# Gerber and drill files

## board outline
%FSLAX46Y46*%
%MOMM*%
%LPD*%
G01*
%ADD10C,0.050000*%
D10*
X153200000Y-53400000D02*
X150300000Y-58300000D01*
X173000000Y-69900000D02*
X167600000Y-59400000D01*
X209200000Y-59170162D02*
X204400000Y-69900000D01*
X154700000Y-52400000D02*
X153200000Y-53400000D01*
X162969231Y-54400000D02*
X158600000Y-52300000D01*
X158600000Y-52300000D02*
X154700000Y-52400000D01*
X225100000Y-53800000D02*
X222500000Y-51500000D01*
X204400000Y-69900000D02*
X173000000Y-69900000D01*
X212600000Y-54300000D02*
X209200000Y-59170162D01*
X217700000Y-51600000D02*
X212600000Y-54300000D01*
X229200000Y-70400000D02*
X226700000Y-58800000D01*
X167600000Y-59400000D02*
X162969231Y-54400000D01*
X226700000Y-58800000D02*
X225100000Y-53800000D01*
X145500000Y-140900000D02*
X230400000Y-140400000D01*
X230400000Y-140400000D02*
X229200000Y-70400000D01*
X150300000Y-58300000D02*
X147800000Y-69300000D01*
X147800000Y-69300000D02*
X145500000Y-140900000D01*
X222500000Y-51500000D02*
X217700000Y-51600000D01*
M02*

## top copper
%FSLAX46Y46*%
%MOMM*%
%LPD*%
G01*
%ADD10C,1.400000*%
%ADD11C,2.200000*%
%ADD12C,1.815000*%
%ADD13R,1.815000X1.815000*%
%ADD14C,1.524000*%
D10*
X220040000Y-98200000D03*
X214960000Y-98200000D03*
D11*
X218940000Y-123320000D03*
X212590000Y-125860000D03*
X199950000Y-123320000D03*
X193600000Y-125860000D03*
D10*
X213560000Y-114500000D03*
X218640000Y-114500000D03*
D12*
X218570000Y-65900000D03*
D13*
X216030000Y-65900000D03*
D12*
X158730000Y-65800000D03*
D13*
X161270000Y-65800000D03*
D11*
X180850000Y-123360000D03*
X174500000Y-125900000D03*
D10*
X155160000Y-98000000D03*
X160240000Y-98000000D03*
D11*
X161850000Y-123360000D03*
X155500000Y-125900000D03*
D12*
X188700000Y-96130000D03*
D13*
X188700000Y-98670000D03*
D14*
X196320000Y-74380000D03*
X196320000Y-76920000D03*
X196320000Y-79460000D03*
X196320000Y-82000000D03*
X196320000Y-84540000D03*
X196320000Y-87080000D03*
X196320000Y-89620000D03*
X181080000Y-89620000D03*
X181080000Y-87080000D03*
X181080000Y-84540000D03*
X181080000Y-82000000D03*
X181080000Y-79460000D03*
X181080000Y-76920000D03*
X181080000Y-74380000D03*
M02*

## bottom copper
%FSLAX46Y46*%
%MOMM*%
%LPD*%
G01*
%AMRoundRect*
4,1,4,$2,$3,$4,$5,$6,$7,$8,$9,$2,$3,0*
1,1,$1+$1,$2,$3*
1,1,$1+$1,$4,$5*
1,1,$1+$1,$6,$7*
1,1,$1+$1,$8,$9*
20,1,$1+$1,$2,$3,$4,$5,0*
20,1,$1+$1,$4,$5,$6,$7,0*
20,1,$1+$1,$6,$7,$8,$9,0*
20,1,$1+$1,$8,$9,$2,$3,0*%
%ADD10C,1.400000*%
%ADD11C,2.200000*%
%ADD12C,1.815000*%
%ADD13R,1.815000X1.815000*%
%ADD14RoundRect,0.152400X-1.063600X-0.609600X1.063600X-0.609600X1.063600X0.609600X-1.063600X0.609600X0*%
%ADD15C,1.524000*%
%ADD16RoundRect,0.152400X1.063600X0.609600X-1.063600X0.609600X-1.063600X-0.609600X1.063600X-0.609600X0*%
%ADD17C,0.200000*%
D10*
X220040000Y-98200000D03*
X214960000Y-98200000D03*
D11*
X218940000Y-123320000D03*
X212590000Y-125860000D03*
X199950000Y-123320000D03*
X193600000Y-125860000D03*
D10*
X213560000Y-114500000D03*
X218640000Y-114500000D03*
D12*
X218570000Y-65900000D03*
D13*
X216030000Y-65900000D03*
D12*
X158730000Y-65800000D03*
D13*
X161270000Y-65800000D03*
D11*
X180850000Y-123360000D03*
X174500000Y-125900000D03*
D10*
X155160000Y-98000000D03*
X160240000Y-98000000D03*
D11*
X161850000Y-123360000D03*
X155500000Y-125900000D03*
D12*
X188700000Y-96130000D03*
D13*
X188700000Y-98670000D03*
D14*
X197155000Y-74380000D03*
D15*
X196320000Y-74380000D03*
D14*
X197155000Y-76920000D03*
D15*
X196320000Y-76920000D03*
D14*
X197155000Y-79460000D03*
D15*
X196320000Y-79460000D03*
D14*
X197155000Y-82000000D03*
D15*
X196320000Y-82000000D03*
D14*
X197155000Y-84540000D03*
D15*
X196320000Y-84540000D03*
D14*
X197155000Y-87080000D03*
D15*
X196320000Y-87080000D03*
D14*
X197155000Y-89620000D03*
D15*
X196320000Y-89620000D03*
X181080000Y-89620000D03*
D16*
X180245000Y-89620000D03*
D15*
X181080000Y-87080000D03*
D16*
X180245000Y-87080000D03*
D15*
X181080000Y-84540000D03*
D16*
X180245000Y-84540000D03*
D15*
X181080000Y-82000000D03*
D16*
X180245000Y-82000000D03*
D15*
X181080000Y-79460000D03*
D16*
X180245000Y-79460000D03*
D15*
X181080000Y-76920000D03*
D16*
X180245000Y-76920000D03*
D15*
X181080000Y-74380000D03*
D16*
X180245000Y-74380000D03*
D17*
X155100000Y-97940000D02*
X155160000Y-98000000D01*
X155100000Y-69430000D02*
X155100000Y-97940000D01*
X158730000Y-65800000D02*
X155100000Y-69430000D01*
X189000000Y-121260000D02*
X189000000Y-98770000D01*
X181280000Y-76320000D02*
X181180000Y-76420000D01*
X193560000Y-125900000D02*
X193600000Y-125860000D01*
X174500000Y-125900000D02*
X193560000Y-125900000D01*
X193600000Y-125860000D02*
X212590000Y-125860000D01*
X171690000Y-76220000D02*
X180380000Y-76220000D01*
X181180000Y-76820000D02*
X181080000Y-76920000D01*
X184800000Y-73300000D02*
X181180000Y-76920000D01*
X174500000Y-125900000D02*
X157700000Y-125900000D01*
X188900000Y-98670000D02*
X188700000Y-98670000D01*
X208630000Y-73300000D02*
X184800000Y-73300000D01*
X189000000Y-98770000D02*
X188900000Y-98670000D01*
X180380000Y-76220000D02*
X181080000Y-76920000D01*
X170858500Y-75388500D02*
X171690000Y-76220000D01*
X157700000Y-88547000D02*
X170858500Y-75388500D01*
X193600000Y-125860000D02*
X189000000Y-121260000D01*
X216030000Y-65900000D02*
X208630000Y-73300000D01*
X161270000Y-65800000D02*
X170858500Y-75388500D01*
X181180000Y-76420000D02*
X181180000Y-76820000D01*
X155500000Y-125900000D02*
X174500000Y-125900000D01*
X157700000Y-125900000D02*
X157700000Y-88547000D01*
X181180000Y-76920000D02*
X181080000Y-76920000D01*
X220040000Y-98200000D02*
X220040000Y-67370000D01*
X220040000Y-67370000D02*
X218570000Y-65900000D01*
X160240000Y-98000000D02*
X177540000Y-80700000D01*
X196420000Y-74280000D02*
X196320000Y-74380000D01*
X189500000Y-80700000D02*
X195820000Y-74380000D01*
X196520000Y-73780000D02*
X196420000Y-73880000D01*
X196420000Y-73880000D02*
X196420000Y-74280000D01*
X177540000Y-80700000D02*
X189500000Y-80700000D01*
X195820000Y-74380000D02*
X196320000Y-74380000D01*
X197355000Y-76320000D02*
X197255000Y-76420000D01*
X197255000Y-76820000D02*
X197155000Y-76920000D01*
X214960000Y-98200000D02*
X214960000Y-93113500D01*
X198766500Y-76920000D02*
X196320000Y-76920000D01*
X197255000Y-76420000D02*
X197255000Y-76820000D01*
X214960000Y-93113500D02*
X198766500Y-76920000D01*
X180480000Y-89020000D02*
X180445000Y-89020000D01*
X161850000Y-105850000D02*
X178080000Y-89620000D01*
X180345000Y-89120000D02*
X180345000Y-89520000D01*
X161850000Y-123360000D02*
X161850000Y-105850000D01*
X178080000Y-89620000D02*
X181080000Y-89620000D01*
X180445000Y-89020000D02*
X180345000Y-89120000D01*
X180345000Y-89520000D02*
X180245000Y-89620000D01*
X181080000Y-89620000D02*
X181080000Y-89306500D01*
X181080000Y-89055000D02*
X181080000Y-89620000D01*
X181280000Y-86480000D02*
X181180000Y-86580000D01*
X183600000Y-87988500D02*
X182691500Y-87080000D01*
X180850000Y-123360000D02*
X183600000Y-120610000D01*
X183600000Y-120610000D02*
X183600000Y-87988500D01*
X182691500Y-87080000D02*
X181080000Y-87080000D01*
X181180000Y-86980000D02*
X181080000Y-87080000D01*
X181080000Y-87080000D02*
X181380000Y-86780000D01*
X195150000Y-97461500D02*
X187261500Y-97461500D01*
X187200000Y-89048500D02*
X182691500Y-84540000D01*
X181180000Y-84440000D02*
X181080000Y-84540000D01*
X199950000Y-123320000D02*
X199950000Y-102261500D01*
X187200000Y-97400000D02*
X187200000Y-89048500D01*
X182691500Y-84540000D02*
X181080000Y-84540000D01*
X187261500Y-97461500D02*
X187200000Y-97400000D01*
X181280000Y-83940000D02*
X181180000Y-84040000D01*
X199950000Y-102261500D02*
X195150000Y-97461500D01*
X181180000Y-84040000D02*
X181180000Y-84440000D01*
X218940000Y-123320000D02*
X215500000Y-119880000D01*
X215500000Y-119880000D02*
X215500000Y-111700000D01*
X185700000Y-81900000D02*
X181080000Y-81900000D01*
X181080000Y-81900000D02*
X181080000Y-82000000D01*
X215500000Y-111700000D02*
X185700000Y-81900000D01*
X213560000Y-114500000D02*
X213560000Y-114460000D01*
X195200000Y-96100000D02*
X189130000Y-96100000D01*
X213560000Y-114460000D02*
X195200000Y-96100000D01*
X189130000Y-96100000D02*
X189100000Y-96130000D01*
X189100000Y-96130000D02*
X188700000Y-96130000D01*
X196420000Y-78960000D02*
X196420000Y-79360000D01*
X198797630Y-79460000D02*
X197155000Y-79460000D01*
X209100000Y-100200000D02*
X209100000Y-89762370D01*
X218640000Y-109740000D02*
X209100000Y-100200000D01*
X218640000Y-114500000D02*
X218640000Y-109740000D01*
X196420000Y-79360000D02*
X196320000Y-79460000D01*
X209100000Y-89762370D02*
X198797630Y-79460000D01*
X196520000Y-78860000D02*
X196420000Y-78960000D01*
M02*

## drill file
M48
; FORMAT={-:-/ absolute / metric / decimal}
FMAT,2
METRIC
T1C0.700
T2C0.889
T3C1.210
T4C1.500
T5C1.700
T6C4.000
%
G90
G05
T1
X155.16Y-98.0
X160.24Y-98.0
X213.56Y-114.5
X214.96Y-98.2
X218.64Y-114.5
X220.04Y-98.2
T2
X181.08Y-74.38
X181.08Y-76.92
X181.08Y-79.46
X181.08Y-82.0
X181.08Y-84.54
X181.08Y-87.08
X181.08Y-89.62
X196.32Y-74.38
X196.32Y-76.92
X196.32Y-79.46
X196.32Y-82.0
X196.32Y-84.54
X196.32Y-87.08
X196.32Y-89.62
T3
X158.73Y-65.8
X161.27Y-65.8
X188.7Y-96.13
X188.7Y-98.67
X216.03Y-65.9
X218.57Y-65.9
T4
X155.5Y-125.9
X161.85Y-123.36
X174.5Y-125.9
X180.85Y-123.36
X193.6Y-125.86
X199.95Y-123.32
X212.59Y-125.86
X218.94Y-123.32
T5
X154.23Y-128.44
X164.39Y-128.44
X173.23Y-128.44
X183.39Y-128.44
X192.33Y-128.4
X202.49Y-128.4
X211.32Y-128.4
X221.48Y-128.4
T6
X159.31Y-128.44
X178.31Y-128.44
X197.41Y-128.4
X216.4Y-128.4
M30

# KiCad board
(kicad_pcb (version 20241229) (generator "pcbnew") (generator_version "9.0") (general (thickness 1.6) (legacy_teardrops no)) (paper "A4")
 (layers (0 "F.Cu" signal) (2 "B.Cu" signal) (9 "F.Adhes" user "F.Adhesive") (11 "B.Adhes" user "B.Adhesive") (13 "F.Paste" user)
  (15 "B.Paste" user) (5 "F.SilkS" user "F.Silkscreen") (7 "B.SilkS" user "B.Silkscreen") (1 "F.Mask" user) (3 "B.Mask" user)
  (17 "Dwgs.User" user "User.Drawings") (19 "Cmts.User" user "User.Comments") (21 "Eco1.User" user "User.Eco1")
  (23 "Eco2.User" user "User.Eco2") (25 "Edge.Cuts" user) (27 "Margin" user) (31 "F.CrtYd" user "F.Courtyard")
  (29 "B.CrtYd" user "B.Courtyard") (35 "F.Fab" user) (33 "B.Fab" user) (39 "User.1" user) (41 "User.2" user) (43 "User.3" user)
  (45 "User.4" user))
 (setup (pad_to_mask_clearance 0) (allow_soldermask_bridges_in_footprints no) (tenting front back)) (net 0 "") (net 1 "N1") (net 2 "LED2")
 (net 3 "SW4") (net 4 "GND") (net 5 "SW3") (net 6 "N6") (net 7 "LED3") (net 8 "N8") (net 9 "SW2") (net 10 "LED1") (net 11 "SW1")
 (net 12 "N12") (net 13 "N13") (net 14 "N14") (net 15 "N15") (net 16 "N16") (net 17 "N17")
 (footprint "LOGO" (layer "F.Cu") (at 164.702705 114.300431)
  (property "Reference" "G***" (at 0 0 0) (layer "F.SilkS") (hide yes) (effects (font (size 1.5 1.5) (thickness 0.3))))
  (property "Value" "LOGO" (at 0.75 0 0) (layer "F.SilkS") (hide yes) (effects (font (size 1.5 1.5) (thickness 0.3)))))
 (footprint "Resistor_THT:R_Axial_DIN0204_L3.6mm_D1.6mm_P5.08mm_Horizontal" (layer "F.Cu") (at 220.04 98.2 180)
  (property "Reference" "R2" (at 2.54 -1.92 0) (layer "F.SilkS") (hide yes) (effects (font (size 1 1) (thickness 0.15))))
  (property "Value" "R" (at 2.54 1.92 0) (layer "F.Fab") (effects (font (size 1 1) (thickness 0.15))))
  (pad "1" thru_hole circle (at 0 0 180) (size 1.4 1.4) (drill 0.7) (layers "*.Cu" "*.Mask") (remove_unused_layers no) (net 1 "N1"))
  (pad "2" thru_hole circle (at 5.08 0 180) (size 1.4 1.4) (drill 0.7) (layers "*.Cu" "*.Mask") (remove_unused_layers no) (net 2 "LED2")))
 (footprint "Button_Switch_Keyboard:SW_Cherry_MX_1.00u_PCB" (layer "F.Cu") (at 218.94 123.32)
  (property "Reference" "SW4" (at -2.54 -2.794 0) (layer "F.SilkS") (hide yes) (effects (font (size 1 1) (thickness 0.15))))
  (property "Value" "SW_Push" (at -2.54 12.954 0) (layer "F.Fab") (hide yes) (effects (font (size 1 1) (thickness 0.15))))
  (pad "" np_thru_hole circle (at -7.62 5.08) (size 1.7 1.7) (drill 1.7) (layers "*.Cu" "*.Mask"))
  (pad "" np_thru_hole circle (at -2.54 5.08) (size 4 4) (drill 4) (layers "*.Cu" "*.Mask"))
  (pad "" np_thru_hole circle (at 2.54 5.08) (size 1.7 1.7) (drill 1.7) (layers "*.Cu" "*.Mask"))
  (pad "1" thru_hole circle (at 0 0) (size 2.2 2.2) (drill 1.5) (layers "*.Cu" "*.Mask") (remove_unused_layers no) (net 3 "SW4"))
  (pad "2" thru_hole circle (at -6.35 2.54) (size 2.2 2.2) (drill 1.5) (layers "*.Cu" "*.Mask") (remove_unused_layers no) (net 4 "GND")))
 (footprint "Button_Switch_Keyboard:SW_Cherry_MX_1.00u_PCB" (layer "F.Cu") (at 199.95 123.32)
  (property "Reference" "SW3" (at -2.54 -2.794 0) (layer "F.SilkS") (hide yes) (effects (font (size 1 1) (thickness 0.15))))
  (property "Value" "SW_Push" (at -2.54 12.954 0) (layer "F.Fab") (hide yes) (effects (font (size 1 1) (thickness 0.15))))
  (pad "" np_thru_hole circle (at -7.62 5.08) (size 1.7 1.7) (drill 1.7) (layers "*.Cu" "*.Mask"))
  (pad "" np_thru_hole circle (at -2.54 5.08) (size 4 4) (drill 4) (layers "*.Cu" "*.Mask"))
  (pad "" np_thru_hole circle (at 2.54 5.08) (size 1.7 1.7) (drill 1.7) (layers "*.Cu" "*.Mask"))
  (pad "1" thru_hole circle (at 0 0) (size 2.2 2.2) (drill 1.5) (layers "*.Cu" "*.Mask") (remove_unused_layers no) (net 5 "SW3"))
  (pad "2" thru_hole circle (at -6.35 2.54) (size 2.2 2.2) (drill 1.5) (layers "*.Cu" "*.Mask") (remove_unused_layers no) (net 4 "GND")))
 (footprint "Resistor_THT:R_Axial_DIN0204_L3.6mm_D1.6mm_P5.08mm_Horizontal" (layer "F.Cu") (at 213.56 114.5)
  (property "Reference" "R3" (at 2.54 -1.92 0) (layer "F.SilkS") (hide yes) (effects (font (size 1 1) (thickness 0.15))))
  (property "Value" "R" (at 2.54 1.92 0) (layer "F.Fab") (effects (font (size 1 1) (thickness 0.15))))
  (pad "1" thru_hole circle (at 0 0) (size 1.4 1.4) (drill 0.7) (layers "*.Cu" "*.Mask") (remove_unused_layers no) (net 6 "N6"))
  (pad "2" thru_hole circle (at 5.08 0) (size 1.4 1.4) (drill 0.7) (layers "*.Cu" "*.Mask") (remove_unused_layers no) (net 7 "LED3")))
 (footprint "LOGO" (layer "F.Cu") (at 189.2 117.3)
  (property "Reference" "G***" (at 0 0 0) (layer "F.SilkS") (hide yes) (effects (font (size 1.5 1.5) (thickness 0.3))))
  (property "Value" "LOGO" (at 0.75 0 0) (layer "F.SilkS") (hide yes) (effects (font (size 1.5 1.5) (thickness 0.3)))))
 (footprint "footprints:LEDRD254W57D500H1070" (layer "F.Cu") (at 217.3 65.9)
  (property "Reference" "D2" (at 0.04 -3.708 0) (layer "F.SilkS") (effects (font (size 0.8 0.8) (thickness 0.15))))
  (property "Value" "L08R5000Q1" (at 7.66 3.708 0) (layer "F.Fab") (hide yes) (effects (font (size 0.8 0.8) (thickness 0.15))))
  (pad "A" thru_hole circle (at 1.27 0) (size 1.815 1.815) (drill 1.21) (layers "*.Cu" "*.Mask") (remove_unused_layers no) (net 1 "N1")
   (solder_mask_margin 0.102))
  (pad "C" thru_hole rect (at -1.27 0) (size 1.815 1.815) (drill 1.21) (layers "*.Cu" "*.Mask") (remove_unused_layers no) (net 4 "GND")
   (solder_mask_margin 0.102)))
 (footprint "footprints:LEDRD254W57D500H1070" (layer "F.Cu") (at 160 65.8 180)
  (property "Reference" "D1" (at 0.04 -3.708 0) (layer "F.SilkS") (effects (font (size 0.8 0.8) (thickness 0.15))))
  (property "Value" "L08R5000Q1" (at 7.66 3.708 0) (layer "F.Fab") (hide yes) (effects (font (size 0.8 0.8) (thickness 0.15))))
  (pad "A" thru_hole circle (at 1.27 0 180) (size 1.815 1.815) (drill 1.21) (layers "*.Cu" "*.Mask") (remove_unused_layers no) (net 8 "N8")
   (solder_mask_margin 0.102))
  (pad "C" thru_hole rect (at -1.27 0 180) (size 1.815 1.815) (drill 1.21) (layers "*.Cu" "*.Mask") (remove_unused_layers no) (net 4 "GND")
   (solder_mask_margin 0.102)))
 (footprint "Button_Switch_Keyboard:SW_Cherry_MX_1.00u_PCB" (layer "F.Cu") (at 180.85 123.36)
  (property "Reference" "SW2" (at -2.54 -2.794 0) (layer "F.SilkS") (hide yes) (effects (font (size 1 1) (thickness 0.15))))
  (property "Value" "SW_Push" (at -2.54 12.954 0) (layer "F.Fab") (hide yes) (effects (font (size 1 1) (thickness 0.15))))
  (pad "" np_thru_hole circle (at -7.62 5.08) (size 1.7 1.7) (drill 1.7) (layers "*.Cu" "*.Mask"))
  (pad "" np_thru_hole circle (at -2.54 5.08) (size 4 4) (drill 4) (layers "*.Cu" "*.Mask"))
  (pad "" np_thru_hole circle (at 2.54 5.08) (size 1.7 1.7) (drill 1.7) (layers "*.Cu" "*.Mask"))
  (pad "1" thru_hole circle (at 0 0) (size 2.2 2.2) (drill 1.5) (layers "*.Cu" "*.Mask") (remove_unused_layers no) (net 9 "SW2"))
  (pad "2" thru_hole circle (at -6.35 2.54) (size 2.2 2.2) (drill 1.5) (layers "*.Cu" "*.Mask") (remove_unused_layers no) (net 4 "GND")))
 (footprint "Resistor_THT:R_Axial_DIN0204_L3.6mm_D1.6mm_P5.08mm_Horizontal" (layer "F.Cu") (at 155.16 98)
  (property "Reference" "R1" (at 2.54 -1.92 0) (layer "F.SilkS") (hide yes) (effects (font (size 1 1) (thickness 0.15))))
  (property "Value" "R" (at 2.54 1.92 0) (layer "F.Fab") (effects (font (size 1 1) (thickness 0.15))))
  (pad "1" thru_hole circle (at 0 0) (size 1.4 1.4) (drill 0.7) (layers "*.Cu" "*.Mask") (remove_unused_layers no) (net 8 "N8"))
  (pad "2" thru_hole circle (at 5.08 0) (size 1.4 1.4) (drill 0.7) (layers "*.Cu" "*.Mask") (remove_unused_layers no) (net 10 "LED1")))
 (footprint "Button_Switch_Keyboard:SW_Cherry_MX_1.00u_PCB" (layer "F.Cu") (at 161.85 123.36)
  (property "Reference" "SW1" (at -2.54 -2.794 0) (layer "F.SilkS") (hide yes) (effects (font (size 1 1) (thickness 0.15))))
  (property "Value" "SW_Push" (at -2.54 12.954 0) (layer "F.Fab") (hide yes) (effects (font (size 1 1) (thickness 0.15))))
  (pad "" np_thru_hole circle (at -7.62 5.08) (size 1.7 1.7) (drill 1.7) (layers "*.Cu" "*.Mask"))
  (pad "" np_thru_hole circle (at -2.54 5.08) (size 4 4) (drill 4) (layers "*.Cu" "*.Mask"))
  (pad "" np_thru_hole circle (at 2.54 5.08) (size 1.7 1.7) (drill 1.7) (layers "*.Cu" "*.Mask"))
  (pad "1" thru_hole circle (at 0 0) (size 2.2 2.2) (drill 1.5) (layers "*.Cu" "*.Mask") (remove_unused_layers no) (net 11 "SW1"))
  (pad "2" thru_hole circle (at -6.35 2.54) (size 2.2 2.2) (drill 1.5) (layers "*.Cu" "*.Mask") (remove_unused_layers no) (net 4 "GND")))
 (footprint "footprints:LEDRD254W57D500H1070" (layer "F.Cu") (at 188.7 97.4 90)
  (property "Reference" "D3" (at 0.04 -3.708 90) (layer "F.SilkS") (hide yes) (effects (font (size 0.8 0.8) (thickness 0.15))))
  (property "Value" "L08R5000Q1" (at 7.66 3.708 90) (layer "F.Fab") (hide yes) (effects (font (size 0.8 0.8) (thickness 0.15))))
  (pad "A" thru_hole circle (at 1.27 0 90) (size 1.815 1.815) (drill 1.21) (layers "*.Cu" "*.Mask") (remove_unused_layers no) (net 6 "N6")
   (solder_mask_margin 0.102))
  (pad "C" thru_hole rect (at -1.27 0 90) (size 1.815 1.815) (drill 1.21) (layers "*.Cu" "*.Mask") (remove_unused_layers no) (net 4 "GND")
   (solder_mask_margin 0.102)))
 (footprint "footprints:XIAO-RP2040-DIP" (layer "B.Cu") (at 188.7 82 180)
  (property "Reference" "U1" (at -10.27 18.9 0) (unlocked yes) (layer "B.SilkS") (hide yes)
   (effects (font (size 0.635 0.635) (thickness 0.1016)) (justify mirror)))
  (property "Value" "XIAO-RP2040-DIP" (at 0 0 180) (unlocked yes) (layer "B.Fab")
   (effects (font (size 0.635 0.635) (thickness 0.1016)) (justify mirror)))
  (pad "1" smd roundrect (at -8.455 7.62) (size 2.432 1.524) (layers "B.Cu" "B.Mask") (roundrect_rratio 0.1) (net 10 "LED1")
   (thermal_bridge_angle 45))
  (pad "1" thru_hole circle (at -7.62 7.62) (size 1.524 1.524) (drill 0.889) (layers "*.Cu" "*.Mask") (remove_unused_layers no)
   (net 10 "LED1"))
  (pad "2" smd roundrect (at -8.455 5.08) (size 2.432 1.524) (layers "B.Cu" "B.Mask") (roundrect_rratio 0.1) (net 2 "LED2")
   (thermal_bridge_angle 45))
  (pad "2" thru_hole circle (at -7.62 5.08) (size 1.524 1.524) (drill 0.889) (layers "*.Cu" "*.Mask") (remove_unused_layers no)
   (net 2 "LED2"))
  (pad "3" smd roundrect (at -8.455 2.54) (size 2.432 1.524) (layers "B.Cu" "B.Mask") (roundrect_rratio 0.1) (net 7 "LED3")
   (thermal_bridge_angle 45))
  (pad "3" thru_hole circle (at -7.62 2.54) (size 1.524 1.524) (drill 0.889) (layers "*.Cu" "*.Mask") (remove_unused_layers no)
   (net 7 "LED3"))
  (pad "4" smd roundrect (at -8.455 0) (size 2.432 1.524) (layers "B.Cu" "B.Mask") (roundrect_rratio 0.1) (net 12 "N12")
   (thermal_bridge_angle 45))
  (pad "4" thru_hole circle (at -7.62 0) (size 1.524 1.524) (drill 0.889) (layers "*.Cu" "*.Mask") (remove_unused_layers no) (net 12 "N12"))
  (pad "5" smd roundrect (at -8.455 -2.54) (size 2.432 1.524) (layers "B.Cu" "B.Mask") (roundrect_rratio 0.1) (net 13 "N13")
   (thermal_bridge_angle 45))
  (pad "5" thru_hole circle (at -7.62 -2.54) (size 1.524 1.524) (drill 0.889) (layers "*.Cu" "*.Mask") (remove_unused_layers no)
   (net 13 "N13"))
  (pad "6" smd roundrect (at -8.455 -5.08) (size 2.432 1.524) (layers "B.Cu" "B.Mask") (roundrect_rratio 0.1) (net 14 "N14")
   (thermal_bridge_angle 45))
  (pad "6" thru_hole circle (at -7.62 -5.08) (size 1.524 1.524) (drill 0.889) (layers "*.Cu" "*.Mask") (remove_unused_layers no)
   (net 14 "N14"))
  (pad "7" smd roundrect (at -8.455 -7.62) (size 2.432 1.524) (layers "B.Cu" "B.Mask") (roundrect_rratio 0.1) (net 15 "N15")
   (thermal_bridge_angle 45))
  (pad "7" thru_hole circle (at -7.62 -7.62) (size 1.524 1.524) (drill 0.889) (layers "*.Cu" "*.Mask") (remove_unused_layers no)
   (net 15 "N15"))
  (pad "8" thru_hole circle (at 7.62 -7.62 180) (size 1.524 1.524) (drill 0.889) (layers "*.Cu" "*.Mask") (remove_unused_layers no)
   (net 11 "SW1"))
  (pad "8" smd roundrect (at 8.455 -7.62 180) (size 2.432 1.524) (layers "B.Cu" "B.Mask") (roundrect_rratio 0.1) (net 11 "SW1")
   (thermal_bridge_angle 45))
  (pad "9" thru_hole circle (at 7.62 -5.08 180) (size 1.524 1.524) (drill 0.889) (layers "*.Cu" "*.Mask") (remove_unused_layers no)
   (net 9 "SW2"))
  (pad "9" smd roundrect (at 8.455 -5.08 180) (size 2.432 1.524) (layers "B.Cu" "B.Mask") (roundrect_rratio 0.1) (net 9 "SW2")
   (thermal_bridge_angle 45))
  (pad "10" thru_hole circle (at 7.62 -2.54 180) (size 1.524 1.524) (drill 0.889) (layers "*.Cu" "*.Mask") (remove_unused_layers no)
   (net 5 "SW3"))
  (pad "10" smd roundrect (at 8.455 -2.54 180) (size 2.432 1.524) (layers "B.Cu" "B.Mask") (roundrect_rratio 0.1) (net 5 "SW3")
   (thermal_bridge_angle 45))
  (pad "11" thru_hole circle (at 7.62 0 180) (size 1.524 1.524) (drill 0.889) (layers "*.Cu" "*.Mask") (remove_unused_layers no)
   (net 3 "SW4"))
  (pad "11" smd roundrect (at 8.455 0 180) (size 2.432 1.524) (layers "B.Cu" "B.Mask") (roundrect_rratio 0.1) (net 3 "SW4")
   (thermal_bridge_angle 45))
  (pad "12" thru_hole circle (at 7.62 2.54 180) (size 1.524 1.524) (drill 0.889) (layers "*.Cu" "*.Mask") (remove_unused_layers no)
   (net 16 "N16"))
  (pad "12" smd roundrect (at 8.455 2.54 180) (size 2.432 1.524) (layers "B.Cu" "B.Mask") (roundrect_rratio 0.1) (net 16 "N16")
   (thermal_bridge_angle 45))
  (pad "13" thru_hole circle (at 7.62 5.08 180) (size 1.524 1.524) (drill 0.889) (layers "*.Cu" "*.Mask") (remove_unused_layers no)
   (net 4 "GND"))
  (pad "13" smd roundrect (at 8.455 5.08 180) (size 2.432 1.524) (layers "B.Cu" "B.Mask") (roundrect_rratio 0.1) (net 4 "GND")
   (thermal_bridge_angle 45))
  (pad "14" thru_hole circle (at 7.62 7.62 180) (size 1.524 1.524) (drill 0.889) (layers "*.Cu" "*.Mask") (remove_unused_layers no)
   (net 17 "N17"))
  (pad "14" smd roundrect (at 8.455 7.62 180) (size 2.432 1.524) (layers "B.Cu" "B.Mask") (roundrect_rratio 0.1) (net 17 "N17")
   (thermal_bridge_angle 45)))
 (gr_line (start 153.2 53.4) (end 150.3 58.3) (stroke (width 0.05) (type default)) (layer "Edge.Cuts"))
 (gr_line (start 173 69.9) (end 167.6 59.4) (stroke (width 0.05) (type default)) (layer "Edge.Cuts"))
 (gr_line (start 209.2 59.170162) (end 204.4 69.9) (stroke (width 0.05) (type default)) (layer "Edge.Cuts"))
 (gr_line (start 154.7 52.4) (end 153.2 53.4) (stroke (width 0.05) (type default)) (layer "Edge.Cuts"))
 (gr_line (start 162.969231 54.4) (end 158.6 52.3) (stroke (width 0.05) (type default)) (layer "Edge.Cuts"))
 (gr_line (start 158.6 52.3) (end 154.7 52.4) (stroke (width 0.05) (type default)) (layer "Edge.Cuts"))
 (gr_line (start 225.1 53.8) (end 222.5 51.5) (stroke (width 0.05) (type default)) (layer "Edge.Cuts"))
 (gr_line (start 204.4 69.9) (end 173 69.9) (stroke (width 0.05) (type default)) (layer "Edge.Cuts"))
 (gr_line (start 212.6 54.3) (end 209.2 59.170162) (stroke (width 0.05) (type default)) (layer "Edge.Cuts"))
 (gr_line (start 217.7 51.6) (end 212.6 54.3) (stroke (width 0.05) (type default)) (layer "Edge.Cuts"))
 (gr_line (start 229.2 70.4) (end 226.7 58.8) (stroke (width 0.05) (type default)) (layer "Edge.Cuts"))
 (gr_line (start 167.6 59.4) (end 162.969231 54.4) (stroke (width 0.05) (type default)) (layer "Edge.Cuts"))
 (gr_line (start 226.7 58.8) (end 225.1 53.8) (stroke (width 0.05) (type solid)) (layer "Edge.Cuts"))
 (gr_line (start 145.5 140.9) (end 230.4 140.4) (stroke (width 0.05) (type default)) (layer "Edge.Cuts"))
 (gr_line (start 230.4 140.4) (end 229.2 70.4) (stroke (width 0.05) (type default)) (layer "Edge.Cuts"))
 (gr_line (start 150.3 58.3) (end 147.8 69.3) (stroke (width 0.05) (type default)) (layer "Edge.Cuts"))
 (gr_line (start 147.8 69.3) (end 145.5 140.9) (stroke (width 0.05) (type default)) (layer "Edge.Cuts"))
 (gr_line (start 222.5 51.5) (end 217.7 51.6) (stroke (width 0.05) (type default)) (layer "Edge.Cuts"))
 (segment (start 155.1 97.94) (end 155.16 98) (width 0.2) (layer "B.Cu") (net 8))
 (segment (start 155.1 69.43) (end 155.1 97.94) (width 0.2) (layer "B.Cu") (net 8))
 (segment (start 158.73 65.8) (end 155.1 69.43) (width 0.2) (layer "B.Cu") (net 8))
 (segment (start 189 121.26) (end 189 98.77) (width 0.2) (layer "B.Cu") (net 4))
 (segment (start 181.28 76.32) (end 181.18 76.42) (width 0.2) (layer "B.Cu") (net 4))
 (segment (start 193.56 125.9) (end 193.6 125.86) (width 0.2) (layer "B.Cu") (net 4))
 (segment (start 174.5 125.9) (end 193.56 125.9) (width 0.2) (layer "B.Cu") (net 4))
 (segment (start 193.6 125.86) (end 212.59 125.86) (width 0.2) (layer "B.Cu") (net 4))
 (segment (start 171.69 76.22) (end 180.38 76.22) (width 0.2) (layer "B.Cu") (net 4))
 (segment (start 181.18 76.82) (end 181.08 76.92) (width 0.2) (layer "B.Cu") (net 4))
 (segment (start 184.8 73.3) (end 181.18 76.92) (width 0.2) (layer "B.Cu") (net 4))
 (segment (start 174.5 125.9) (end 157.7 125.9) (width 0.2) (layer "B.Cu") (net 4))
 (segment (start 188.9 98.67) (end 188.7 98.67) (width 0.2) (layer "B.Cu") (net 4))
 (segment (start 208.63 73.3) (end 184.8 73.3) (width 0.2) (layer "B.Cu") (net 4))
 (segment (start 189 98.77) (end 188.9 98.67) (width 0.2) (layer "B.Cu") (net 4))
 (segment (start 180.38 76.22) (end 181.08 76.92) (width 0.2) (layer "B.Cu") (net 4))
 (segment (start 170.8585 75.3885) (end 171.69 76.22) (width 0.2) (layer "B.Cu") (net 4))
 (segment (start 157.7 88.547) (end 170.8585 75.3885) (width 0.2) (layer "B.Cu") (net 4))
 (segment (start 193.6 125.86) (end 189 121.26) (width 0.2) (layer "B.Cu") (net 4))
 (segment (start 216.03 65.9) (end 208.63 73.3) (width 0.2) (layer "B.Cu") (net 4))
 (segment (start 161.27 65.8) (end 170.8585 75.3885) (width 0.2) (layer "B.Cu") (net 4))
 (segment (start 181.18 76.42) (end 181.18 76.82) (width 0.2) (layer "B.Cu") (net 4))
 (segment (start 155.5 125.9) (end 174.5 125.9) (width 0.2) (layer "B.Cu") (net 4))
 (segment (start 157.7 125.9) (end 157.7 88.547) (width 0.2) (layer "B.Cu") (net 4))
 (segment (start 181.18 76.92) (end 181.08 76.92) (width 0.2) (layer "B.Cu") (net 4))
 (segment (start 220.04 98.2) (end 220.04 67.37) (width 0.2) (layer "B.Cu") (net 1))
 (segment (start 220.04 67.37) (end 218.57 65.9) (width 0.2) (layer "B.Cu") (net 1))
 (segment (start 160.24 98) (end 177.54 80.7) (width 0.2) (layer "B.Cu") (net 10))
 (segment (start 196.42 74.28) (end 196.32 74.38) (width 0.2) (layer "B.Cu") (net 10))
 (segment (start 189.5 80.7) (end 195.82 74.38) (width 0.2) (layer "B.Cu") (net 10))
 (segment (start 196.52 73.78) (end 196.42 73.88) (width 0.2) (layer "B.Cu") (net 10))
 (segment (start 196.42 73.88) (end 196.42 74.28) (width 0.2) (layer "B.Cu") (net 10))
 (segment (start 177.54 80.7) (end 189.5 80.7) (width 0.2) (layer "B.Cu") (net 10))
 (segment (start 195.82 74.38) (end 196.32 74.38) (width 0.2) (layer "B.Cu") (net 10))
 (segment (start 197.355 76.32) (end 197.255 76.42) (width 0.2) (layer "B.Cu") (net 2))
 (segment (start 197.255 76.82) (end 197.155 76.92) (width 0.2) (layer "B.Cu") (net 2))
 (segment (start 214.96 98.2) (end 214.96 93.1135) (width 0.2) (layer "B.Cu") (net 2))
 (segment (start 198.7665 76.92) (end 196.32 76.92) (width 0.2) (layer "B.Cu") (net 2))
 (segment (start 197.255 76.42) (end 197.255 76.82) (width 0.2) (layer "B.Cu") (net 2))
 (segment (start 214.96 93.1135) (end 198.7665 76.92) (width 0.2) (layer "B.Cu") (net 2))
 (segment (start 180.48 89.02) (end 180.445 89.02) (width 0.2) (layer "B.Cu") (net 11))
 (segment (start 161.85 105.85) (end 178.08 89.62) (width 0.2) (layer "B.Cu") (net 11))
 (segment (start 180.345 89.12) (end 180.345 89.52) (width 0.2) (layer "B.Cu") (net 11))
 (segment (start 161.85 123.36) (end 161.85 105.85) (width 0.2) (layer "B.Cu") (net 11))
 (segment (start 178.08 89.62) (end 181.08 89.62) (width 0.2) (layer "B.Cu") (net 11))
 (segment (start 180.445 89.02) (end 180.345 89.12) (width 0.2) (layer "B.Cu") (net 11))
 (segment (start 180.345 89.52) (end 180.245 89.62) (width 0.2) (layer "B.Cu") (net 11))
 (segment (start 181.08 89.62) (end 181.08 89.3065) (width 0.2) (layer "B.Cu") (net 11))
 (segment (start 181.08 89.055) (end 181.08 89.62) (width 0.2) (layer "B.Cu") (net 11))
 (segment (start 181.28 86.48) (end 181.18 86.58) (width 0.2) (layer "B.Cu") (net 9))
 (segment (start 183.6 87.9885) (end 182.6915 87.08) (width 0.2) (layer "B.Cu") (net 9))
 (segment (start 180.85 123.36) (end 183.6 120.61) (width 0.2) (layer "B.Cu") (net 9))
 (segment (start 183.6 120.61) (end 183.6 87.9885) (width 0.2) (layer "B.Cu") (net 9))
 (segment (start 182.6915 87.08) (end 181.08 87.08) (width 0.2) (layer "B.Cu") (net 9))
 (segment (start 181.18 86.98) (end 181.08 87.08) (width 0.2) (layer "B.Cu") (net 9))
 (segment (start 181.08 87.08) (end 181.38 86.78) (width 0.2) (layer "B.Cu") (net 9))
 (segment (start 195.15 97.4615) (end 187.2615 97.4615) (width 0.2) (layer "B.Cu") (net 5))
 (segment (start 187.2 89.0485) (end 182.6915 84.54) (width 0.2) (layer "B.Cu") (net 5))
 (segment (start 181.18 84.44) (end 181.08 84.54) (width 0.2) (layer "B.Cu") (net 5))
 (segment (start 199.95 123.32) (end 199.95 102.2615) (width 0.2) (layer "B.Cu") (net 5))
 (segment (start 187.2 97.4) (end 187.2 89.0485) (width 0.2) (layer "B.Cu") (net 5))
 (segment (start 182.6915 84.54) (end 181.08 84.54) (width 0.2) (layer "B.Cu") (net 5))
 (segment (start 187.2615 97.4615) (end 187.2 97.4) (width 0.2) (layer "B.Cu") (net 5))
 (segment (start 181.28 83.94) (end 181.18 84.04) (width 0.2) (layer "B.Cu") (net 5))
 (segment (start 199.95 102.2615) (end 195.15 97.4615) (width 0.2) (layer "B.Cu") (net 5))
 (segment (start 181.18 84.04) (end 181.18 84.44) (width 0.2) (layer "B.Cu") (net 5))
 (segment (start 218.94 123.32) (end 215.5 119.88) (width 0.2) (layer "B.Cu") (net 3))
 (segment (start 215.5 119.88) (end 215.5 111.7) (width 0.2) (layer "B.Cu") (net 3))
 (segment (start 185.7 81.9) (end 181.08 81.9) (width 0.2) (layer "B.Cu") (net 3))
 (segment (start 181.08 81.9) (end 181.08 82) (width 0.2) (layer "B.Cu") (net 3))
 (segment (start 215.5 111.7) (end 185.7 81.9) (width 0.2) (layer "B.Cu") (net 3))
 (segment (start 213.56 114.5) (end 213.56 114.46) (width 0.2) (layer "B.Cu") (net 6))
 (segment (start 195.2 96.1) (end 189.13 96.1) (width 0.2) (layer "B.Cu") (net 6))
 (segment (start 213.56 114.46) (end 195.2 96.1) (width 0.2) (layer "B.Cu") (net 6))
 (segment (start 189.13 96.1) (end 189.1 96.13) (width 0.2) (layer "B.Cu") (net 6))
 (segment (start 189.1 96.13) (end 188.7 96.13) (width 0.2) (layer "B.Cu") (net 6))
 (segment (start 196.42 78.96) (end 196.42 79.36) (width 0.2) (layer "B.Cu") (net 7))
 (segment (start 198.79763 79.46) (end 197.155 79.46) (width 0.2) (layer "B.Cu") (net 7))
 (segment (start 209.1 100.2) (end 209.1 89.76237) (width 0.2) (layer "B.Cu") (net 7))
 (segment (start 218.64 109.74) (end 209.1 100.2) (width 0.2) (layer "B.Cu") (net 7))
 (segment (start 218.64 114.5) (end 218.64 109.74) (width 0.2) (layer "B.Cu") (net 7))
 (segment (start 196.42 79.36) (end 196.32 79.46) (width 0.2) (layer "B.Cu") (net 7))
 (segment (start 209.1 89.76237) (end 198.79763 79.46) (width 0.2) (layer "B.Cu") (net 7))
 (segment (start 196.52 78.86) (end 196.42 78.96) (width 0.2) (layer "B.Cu") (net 7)))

